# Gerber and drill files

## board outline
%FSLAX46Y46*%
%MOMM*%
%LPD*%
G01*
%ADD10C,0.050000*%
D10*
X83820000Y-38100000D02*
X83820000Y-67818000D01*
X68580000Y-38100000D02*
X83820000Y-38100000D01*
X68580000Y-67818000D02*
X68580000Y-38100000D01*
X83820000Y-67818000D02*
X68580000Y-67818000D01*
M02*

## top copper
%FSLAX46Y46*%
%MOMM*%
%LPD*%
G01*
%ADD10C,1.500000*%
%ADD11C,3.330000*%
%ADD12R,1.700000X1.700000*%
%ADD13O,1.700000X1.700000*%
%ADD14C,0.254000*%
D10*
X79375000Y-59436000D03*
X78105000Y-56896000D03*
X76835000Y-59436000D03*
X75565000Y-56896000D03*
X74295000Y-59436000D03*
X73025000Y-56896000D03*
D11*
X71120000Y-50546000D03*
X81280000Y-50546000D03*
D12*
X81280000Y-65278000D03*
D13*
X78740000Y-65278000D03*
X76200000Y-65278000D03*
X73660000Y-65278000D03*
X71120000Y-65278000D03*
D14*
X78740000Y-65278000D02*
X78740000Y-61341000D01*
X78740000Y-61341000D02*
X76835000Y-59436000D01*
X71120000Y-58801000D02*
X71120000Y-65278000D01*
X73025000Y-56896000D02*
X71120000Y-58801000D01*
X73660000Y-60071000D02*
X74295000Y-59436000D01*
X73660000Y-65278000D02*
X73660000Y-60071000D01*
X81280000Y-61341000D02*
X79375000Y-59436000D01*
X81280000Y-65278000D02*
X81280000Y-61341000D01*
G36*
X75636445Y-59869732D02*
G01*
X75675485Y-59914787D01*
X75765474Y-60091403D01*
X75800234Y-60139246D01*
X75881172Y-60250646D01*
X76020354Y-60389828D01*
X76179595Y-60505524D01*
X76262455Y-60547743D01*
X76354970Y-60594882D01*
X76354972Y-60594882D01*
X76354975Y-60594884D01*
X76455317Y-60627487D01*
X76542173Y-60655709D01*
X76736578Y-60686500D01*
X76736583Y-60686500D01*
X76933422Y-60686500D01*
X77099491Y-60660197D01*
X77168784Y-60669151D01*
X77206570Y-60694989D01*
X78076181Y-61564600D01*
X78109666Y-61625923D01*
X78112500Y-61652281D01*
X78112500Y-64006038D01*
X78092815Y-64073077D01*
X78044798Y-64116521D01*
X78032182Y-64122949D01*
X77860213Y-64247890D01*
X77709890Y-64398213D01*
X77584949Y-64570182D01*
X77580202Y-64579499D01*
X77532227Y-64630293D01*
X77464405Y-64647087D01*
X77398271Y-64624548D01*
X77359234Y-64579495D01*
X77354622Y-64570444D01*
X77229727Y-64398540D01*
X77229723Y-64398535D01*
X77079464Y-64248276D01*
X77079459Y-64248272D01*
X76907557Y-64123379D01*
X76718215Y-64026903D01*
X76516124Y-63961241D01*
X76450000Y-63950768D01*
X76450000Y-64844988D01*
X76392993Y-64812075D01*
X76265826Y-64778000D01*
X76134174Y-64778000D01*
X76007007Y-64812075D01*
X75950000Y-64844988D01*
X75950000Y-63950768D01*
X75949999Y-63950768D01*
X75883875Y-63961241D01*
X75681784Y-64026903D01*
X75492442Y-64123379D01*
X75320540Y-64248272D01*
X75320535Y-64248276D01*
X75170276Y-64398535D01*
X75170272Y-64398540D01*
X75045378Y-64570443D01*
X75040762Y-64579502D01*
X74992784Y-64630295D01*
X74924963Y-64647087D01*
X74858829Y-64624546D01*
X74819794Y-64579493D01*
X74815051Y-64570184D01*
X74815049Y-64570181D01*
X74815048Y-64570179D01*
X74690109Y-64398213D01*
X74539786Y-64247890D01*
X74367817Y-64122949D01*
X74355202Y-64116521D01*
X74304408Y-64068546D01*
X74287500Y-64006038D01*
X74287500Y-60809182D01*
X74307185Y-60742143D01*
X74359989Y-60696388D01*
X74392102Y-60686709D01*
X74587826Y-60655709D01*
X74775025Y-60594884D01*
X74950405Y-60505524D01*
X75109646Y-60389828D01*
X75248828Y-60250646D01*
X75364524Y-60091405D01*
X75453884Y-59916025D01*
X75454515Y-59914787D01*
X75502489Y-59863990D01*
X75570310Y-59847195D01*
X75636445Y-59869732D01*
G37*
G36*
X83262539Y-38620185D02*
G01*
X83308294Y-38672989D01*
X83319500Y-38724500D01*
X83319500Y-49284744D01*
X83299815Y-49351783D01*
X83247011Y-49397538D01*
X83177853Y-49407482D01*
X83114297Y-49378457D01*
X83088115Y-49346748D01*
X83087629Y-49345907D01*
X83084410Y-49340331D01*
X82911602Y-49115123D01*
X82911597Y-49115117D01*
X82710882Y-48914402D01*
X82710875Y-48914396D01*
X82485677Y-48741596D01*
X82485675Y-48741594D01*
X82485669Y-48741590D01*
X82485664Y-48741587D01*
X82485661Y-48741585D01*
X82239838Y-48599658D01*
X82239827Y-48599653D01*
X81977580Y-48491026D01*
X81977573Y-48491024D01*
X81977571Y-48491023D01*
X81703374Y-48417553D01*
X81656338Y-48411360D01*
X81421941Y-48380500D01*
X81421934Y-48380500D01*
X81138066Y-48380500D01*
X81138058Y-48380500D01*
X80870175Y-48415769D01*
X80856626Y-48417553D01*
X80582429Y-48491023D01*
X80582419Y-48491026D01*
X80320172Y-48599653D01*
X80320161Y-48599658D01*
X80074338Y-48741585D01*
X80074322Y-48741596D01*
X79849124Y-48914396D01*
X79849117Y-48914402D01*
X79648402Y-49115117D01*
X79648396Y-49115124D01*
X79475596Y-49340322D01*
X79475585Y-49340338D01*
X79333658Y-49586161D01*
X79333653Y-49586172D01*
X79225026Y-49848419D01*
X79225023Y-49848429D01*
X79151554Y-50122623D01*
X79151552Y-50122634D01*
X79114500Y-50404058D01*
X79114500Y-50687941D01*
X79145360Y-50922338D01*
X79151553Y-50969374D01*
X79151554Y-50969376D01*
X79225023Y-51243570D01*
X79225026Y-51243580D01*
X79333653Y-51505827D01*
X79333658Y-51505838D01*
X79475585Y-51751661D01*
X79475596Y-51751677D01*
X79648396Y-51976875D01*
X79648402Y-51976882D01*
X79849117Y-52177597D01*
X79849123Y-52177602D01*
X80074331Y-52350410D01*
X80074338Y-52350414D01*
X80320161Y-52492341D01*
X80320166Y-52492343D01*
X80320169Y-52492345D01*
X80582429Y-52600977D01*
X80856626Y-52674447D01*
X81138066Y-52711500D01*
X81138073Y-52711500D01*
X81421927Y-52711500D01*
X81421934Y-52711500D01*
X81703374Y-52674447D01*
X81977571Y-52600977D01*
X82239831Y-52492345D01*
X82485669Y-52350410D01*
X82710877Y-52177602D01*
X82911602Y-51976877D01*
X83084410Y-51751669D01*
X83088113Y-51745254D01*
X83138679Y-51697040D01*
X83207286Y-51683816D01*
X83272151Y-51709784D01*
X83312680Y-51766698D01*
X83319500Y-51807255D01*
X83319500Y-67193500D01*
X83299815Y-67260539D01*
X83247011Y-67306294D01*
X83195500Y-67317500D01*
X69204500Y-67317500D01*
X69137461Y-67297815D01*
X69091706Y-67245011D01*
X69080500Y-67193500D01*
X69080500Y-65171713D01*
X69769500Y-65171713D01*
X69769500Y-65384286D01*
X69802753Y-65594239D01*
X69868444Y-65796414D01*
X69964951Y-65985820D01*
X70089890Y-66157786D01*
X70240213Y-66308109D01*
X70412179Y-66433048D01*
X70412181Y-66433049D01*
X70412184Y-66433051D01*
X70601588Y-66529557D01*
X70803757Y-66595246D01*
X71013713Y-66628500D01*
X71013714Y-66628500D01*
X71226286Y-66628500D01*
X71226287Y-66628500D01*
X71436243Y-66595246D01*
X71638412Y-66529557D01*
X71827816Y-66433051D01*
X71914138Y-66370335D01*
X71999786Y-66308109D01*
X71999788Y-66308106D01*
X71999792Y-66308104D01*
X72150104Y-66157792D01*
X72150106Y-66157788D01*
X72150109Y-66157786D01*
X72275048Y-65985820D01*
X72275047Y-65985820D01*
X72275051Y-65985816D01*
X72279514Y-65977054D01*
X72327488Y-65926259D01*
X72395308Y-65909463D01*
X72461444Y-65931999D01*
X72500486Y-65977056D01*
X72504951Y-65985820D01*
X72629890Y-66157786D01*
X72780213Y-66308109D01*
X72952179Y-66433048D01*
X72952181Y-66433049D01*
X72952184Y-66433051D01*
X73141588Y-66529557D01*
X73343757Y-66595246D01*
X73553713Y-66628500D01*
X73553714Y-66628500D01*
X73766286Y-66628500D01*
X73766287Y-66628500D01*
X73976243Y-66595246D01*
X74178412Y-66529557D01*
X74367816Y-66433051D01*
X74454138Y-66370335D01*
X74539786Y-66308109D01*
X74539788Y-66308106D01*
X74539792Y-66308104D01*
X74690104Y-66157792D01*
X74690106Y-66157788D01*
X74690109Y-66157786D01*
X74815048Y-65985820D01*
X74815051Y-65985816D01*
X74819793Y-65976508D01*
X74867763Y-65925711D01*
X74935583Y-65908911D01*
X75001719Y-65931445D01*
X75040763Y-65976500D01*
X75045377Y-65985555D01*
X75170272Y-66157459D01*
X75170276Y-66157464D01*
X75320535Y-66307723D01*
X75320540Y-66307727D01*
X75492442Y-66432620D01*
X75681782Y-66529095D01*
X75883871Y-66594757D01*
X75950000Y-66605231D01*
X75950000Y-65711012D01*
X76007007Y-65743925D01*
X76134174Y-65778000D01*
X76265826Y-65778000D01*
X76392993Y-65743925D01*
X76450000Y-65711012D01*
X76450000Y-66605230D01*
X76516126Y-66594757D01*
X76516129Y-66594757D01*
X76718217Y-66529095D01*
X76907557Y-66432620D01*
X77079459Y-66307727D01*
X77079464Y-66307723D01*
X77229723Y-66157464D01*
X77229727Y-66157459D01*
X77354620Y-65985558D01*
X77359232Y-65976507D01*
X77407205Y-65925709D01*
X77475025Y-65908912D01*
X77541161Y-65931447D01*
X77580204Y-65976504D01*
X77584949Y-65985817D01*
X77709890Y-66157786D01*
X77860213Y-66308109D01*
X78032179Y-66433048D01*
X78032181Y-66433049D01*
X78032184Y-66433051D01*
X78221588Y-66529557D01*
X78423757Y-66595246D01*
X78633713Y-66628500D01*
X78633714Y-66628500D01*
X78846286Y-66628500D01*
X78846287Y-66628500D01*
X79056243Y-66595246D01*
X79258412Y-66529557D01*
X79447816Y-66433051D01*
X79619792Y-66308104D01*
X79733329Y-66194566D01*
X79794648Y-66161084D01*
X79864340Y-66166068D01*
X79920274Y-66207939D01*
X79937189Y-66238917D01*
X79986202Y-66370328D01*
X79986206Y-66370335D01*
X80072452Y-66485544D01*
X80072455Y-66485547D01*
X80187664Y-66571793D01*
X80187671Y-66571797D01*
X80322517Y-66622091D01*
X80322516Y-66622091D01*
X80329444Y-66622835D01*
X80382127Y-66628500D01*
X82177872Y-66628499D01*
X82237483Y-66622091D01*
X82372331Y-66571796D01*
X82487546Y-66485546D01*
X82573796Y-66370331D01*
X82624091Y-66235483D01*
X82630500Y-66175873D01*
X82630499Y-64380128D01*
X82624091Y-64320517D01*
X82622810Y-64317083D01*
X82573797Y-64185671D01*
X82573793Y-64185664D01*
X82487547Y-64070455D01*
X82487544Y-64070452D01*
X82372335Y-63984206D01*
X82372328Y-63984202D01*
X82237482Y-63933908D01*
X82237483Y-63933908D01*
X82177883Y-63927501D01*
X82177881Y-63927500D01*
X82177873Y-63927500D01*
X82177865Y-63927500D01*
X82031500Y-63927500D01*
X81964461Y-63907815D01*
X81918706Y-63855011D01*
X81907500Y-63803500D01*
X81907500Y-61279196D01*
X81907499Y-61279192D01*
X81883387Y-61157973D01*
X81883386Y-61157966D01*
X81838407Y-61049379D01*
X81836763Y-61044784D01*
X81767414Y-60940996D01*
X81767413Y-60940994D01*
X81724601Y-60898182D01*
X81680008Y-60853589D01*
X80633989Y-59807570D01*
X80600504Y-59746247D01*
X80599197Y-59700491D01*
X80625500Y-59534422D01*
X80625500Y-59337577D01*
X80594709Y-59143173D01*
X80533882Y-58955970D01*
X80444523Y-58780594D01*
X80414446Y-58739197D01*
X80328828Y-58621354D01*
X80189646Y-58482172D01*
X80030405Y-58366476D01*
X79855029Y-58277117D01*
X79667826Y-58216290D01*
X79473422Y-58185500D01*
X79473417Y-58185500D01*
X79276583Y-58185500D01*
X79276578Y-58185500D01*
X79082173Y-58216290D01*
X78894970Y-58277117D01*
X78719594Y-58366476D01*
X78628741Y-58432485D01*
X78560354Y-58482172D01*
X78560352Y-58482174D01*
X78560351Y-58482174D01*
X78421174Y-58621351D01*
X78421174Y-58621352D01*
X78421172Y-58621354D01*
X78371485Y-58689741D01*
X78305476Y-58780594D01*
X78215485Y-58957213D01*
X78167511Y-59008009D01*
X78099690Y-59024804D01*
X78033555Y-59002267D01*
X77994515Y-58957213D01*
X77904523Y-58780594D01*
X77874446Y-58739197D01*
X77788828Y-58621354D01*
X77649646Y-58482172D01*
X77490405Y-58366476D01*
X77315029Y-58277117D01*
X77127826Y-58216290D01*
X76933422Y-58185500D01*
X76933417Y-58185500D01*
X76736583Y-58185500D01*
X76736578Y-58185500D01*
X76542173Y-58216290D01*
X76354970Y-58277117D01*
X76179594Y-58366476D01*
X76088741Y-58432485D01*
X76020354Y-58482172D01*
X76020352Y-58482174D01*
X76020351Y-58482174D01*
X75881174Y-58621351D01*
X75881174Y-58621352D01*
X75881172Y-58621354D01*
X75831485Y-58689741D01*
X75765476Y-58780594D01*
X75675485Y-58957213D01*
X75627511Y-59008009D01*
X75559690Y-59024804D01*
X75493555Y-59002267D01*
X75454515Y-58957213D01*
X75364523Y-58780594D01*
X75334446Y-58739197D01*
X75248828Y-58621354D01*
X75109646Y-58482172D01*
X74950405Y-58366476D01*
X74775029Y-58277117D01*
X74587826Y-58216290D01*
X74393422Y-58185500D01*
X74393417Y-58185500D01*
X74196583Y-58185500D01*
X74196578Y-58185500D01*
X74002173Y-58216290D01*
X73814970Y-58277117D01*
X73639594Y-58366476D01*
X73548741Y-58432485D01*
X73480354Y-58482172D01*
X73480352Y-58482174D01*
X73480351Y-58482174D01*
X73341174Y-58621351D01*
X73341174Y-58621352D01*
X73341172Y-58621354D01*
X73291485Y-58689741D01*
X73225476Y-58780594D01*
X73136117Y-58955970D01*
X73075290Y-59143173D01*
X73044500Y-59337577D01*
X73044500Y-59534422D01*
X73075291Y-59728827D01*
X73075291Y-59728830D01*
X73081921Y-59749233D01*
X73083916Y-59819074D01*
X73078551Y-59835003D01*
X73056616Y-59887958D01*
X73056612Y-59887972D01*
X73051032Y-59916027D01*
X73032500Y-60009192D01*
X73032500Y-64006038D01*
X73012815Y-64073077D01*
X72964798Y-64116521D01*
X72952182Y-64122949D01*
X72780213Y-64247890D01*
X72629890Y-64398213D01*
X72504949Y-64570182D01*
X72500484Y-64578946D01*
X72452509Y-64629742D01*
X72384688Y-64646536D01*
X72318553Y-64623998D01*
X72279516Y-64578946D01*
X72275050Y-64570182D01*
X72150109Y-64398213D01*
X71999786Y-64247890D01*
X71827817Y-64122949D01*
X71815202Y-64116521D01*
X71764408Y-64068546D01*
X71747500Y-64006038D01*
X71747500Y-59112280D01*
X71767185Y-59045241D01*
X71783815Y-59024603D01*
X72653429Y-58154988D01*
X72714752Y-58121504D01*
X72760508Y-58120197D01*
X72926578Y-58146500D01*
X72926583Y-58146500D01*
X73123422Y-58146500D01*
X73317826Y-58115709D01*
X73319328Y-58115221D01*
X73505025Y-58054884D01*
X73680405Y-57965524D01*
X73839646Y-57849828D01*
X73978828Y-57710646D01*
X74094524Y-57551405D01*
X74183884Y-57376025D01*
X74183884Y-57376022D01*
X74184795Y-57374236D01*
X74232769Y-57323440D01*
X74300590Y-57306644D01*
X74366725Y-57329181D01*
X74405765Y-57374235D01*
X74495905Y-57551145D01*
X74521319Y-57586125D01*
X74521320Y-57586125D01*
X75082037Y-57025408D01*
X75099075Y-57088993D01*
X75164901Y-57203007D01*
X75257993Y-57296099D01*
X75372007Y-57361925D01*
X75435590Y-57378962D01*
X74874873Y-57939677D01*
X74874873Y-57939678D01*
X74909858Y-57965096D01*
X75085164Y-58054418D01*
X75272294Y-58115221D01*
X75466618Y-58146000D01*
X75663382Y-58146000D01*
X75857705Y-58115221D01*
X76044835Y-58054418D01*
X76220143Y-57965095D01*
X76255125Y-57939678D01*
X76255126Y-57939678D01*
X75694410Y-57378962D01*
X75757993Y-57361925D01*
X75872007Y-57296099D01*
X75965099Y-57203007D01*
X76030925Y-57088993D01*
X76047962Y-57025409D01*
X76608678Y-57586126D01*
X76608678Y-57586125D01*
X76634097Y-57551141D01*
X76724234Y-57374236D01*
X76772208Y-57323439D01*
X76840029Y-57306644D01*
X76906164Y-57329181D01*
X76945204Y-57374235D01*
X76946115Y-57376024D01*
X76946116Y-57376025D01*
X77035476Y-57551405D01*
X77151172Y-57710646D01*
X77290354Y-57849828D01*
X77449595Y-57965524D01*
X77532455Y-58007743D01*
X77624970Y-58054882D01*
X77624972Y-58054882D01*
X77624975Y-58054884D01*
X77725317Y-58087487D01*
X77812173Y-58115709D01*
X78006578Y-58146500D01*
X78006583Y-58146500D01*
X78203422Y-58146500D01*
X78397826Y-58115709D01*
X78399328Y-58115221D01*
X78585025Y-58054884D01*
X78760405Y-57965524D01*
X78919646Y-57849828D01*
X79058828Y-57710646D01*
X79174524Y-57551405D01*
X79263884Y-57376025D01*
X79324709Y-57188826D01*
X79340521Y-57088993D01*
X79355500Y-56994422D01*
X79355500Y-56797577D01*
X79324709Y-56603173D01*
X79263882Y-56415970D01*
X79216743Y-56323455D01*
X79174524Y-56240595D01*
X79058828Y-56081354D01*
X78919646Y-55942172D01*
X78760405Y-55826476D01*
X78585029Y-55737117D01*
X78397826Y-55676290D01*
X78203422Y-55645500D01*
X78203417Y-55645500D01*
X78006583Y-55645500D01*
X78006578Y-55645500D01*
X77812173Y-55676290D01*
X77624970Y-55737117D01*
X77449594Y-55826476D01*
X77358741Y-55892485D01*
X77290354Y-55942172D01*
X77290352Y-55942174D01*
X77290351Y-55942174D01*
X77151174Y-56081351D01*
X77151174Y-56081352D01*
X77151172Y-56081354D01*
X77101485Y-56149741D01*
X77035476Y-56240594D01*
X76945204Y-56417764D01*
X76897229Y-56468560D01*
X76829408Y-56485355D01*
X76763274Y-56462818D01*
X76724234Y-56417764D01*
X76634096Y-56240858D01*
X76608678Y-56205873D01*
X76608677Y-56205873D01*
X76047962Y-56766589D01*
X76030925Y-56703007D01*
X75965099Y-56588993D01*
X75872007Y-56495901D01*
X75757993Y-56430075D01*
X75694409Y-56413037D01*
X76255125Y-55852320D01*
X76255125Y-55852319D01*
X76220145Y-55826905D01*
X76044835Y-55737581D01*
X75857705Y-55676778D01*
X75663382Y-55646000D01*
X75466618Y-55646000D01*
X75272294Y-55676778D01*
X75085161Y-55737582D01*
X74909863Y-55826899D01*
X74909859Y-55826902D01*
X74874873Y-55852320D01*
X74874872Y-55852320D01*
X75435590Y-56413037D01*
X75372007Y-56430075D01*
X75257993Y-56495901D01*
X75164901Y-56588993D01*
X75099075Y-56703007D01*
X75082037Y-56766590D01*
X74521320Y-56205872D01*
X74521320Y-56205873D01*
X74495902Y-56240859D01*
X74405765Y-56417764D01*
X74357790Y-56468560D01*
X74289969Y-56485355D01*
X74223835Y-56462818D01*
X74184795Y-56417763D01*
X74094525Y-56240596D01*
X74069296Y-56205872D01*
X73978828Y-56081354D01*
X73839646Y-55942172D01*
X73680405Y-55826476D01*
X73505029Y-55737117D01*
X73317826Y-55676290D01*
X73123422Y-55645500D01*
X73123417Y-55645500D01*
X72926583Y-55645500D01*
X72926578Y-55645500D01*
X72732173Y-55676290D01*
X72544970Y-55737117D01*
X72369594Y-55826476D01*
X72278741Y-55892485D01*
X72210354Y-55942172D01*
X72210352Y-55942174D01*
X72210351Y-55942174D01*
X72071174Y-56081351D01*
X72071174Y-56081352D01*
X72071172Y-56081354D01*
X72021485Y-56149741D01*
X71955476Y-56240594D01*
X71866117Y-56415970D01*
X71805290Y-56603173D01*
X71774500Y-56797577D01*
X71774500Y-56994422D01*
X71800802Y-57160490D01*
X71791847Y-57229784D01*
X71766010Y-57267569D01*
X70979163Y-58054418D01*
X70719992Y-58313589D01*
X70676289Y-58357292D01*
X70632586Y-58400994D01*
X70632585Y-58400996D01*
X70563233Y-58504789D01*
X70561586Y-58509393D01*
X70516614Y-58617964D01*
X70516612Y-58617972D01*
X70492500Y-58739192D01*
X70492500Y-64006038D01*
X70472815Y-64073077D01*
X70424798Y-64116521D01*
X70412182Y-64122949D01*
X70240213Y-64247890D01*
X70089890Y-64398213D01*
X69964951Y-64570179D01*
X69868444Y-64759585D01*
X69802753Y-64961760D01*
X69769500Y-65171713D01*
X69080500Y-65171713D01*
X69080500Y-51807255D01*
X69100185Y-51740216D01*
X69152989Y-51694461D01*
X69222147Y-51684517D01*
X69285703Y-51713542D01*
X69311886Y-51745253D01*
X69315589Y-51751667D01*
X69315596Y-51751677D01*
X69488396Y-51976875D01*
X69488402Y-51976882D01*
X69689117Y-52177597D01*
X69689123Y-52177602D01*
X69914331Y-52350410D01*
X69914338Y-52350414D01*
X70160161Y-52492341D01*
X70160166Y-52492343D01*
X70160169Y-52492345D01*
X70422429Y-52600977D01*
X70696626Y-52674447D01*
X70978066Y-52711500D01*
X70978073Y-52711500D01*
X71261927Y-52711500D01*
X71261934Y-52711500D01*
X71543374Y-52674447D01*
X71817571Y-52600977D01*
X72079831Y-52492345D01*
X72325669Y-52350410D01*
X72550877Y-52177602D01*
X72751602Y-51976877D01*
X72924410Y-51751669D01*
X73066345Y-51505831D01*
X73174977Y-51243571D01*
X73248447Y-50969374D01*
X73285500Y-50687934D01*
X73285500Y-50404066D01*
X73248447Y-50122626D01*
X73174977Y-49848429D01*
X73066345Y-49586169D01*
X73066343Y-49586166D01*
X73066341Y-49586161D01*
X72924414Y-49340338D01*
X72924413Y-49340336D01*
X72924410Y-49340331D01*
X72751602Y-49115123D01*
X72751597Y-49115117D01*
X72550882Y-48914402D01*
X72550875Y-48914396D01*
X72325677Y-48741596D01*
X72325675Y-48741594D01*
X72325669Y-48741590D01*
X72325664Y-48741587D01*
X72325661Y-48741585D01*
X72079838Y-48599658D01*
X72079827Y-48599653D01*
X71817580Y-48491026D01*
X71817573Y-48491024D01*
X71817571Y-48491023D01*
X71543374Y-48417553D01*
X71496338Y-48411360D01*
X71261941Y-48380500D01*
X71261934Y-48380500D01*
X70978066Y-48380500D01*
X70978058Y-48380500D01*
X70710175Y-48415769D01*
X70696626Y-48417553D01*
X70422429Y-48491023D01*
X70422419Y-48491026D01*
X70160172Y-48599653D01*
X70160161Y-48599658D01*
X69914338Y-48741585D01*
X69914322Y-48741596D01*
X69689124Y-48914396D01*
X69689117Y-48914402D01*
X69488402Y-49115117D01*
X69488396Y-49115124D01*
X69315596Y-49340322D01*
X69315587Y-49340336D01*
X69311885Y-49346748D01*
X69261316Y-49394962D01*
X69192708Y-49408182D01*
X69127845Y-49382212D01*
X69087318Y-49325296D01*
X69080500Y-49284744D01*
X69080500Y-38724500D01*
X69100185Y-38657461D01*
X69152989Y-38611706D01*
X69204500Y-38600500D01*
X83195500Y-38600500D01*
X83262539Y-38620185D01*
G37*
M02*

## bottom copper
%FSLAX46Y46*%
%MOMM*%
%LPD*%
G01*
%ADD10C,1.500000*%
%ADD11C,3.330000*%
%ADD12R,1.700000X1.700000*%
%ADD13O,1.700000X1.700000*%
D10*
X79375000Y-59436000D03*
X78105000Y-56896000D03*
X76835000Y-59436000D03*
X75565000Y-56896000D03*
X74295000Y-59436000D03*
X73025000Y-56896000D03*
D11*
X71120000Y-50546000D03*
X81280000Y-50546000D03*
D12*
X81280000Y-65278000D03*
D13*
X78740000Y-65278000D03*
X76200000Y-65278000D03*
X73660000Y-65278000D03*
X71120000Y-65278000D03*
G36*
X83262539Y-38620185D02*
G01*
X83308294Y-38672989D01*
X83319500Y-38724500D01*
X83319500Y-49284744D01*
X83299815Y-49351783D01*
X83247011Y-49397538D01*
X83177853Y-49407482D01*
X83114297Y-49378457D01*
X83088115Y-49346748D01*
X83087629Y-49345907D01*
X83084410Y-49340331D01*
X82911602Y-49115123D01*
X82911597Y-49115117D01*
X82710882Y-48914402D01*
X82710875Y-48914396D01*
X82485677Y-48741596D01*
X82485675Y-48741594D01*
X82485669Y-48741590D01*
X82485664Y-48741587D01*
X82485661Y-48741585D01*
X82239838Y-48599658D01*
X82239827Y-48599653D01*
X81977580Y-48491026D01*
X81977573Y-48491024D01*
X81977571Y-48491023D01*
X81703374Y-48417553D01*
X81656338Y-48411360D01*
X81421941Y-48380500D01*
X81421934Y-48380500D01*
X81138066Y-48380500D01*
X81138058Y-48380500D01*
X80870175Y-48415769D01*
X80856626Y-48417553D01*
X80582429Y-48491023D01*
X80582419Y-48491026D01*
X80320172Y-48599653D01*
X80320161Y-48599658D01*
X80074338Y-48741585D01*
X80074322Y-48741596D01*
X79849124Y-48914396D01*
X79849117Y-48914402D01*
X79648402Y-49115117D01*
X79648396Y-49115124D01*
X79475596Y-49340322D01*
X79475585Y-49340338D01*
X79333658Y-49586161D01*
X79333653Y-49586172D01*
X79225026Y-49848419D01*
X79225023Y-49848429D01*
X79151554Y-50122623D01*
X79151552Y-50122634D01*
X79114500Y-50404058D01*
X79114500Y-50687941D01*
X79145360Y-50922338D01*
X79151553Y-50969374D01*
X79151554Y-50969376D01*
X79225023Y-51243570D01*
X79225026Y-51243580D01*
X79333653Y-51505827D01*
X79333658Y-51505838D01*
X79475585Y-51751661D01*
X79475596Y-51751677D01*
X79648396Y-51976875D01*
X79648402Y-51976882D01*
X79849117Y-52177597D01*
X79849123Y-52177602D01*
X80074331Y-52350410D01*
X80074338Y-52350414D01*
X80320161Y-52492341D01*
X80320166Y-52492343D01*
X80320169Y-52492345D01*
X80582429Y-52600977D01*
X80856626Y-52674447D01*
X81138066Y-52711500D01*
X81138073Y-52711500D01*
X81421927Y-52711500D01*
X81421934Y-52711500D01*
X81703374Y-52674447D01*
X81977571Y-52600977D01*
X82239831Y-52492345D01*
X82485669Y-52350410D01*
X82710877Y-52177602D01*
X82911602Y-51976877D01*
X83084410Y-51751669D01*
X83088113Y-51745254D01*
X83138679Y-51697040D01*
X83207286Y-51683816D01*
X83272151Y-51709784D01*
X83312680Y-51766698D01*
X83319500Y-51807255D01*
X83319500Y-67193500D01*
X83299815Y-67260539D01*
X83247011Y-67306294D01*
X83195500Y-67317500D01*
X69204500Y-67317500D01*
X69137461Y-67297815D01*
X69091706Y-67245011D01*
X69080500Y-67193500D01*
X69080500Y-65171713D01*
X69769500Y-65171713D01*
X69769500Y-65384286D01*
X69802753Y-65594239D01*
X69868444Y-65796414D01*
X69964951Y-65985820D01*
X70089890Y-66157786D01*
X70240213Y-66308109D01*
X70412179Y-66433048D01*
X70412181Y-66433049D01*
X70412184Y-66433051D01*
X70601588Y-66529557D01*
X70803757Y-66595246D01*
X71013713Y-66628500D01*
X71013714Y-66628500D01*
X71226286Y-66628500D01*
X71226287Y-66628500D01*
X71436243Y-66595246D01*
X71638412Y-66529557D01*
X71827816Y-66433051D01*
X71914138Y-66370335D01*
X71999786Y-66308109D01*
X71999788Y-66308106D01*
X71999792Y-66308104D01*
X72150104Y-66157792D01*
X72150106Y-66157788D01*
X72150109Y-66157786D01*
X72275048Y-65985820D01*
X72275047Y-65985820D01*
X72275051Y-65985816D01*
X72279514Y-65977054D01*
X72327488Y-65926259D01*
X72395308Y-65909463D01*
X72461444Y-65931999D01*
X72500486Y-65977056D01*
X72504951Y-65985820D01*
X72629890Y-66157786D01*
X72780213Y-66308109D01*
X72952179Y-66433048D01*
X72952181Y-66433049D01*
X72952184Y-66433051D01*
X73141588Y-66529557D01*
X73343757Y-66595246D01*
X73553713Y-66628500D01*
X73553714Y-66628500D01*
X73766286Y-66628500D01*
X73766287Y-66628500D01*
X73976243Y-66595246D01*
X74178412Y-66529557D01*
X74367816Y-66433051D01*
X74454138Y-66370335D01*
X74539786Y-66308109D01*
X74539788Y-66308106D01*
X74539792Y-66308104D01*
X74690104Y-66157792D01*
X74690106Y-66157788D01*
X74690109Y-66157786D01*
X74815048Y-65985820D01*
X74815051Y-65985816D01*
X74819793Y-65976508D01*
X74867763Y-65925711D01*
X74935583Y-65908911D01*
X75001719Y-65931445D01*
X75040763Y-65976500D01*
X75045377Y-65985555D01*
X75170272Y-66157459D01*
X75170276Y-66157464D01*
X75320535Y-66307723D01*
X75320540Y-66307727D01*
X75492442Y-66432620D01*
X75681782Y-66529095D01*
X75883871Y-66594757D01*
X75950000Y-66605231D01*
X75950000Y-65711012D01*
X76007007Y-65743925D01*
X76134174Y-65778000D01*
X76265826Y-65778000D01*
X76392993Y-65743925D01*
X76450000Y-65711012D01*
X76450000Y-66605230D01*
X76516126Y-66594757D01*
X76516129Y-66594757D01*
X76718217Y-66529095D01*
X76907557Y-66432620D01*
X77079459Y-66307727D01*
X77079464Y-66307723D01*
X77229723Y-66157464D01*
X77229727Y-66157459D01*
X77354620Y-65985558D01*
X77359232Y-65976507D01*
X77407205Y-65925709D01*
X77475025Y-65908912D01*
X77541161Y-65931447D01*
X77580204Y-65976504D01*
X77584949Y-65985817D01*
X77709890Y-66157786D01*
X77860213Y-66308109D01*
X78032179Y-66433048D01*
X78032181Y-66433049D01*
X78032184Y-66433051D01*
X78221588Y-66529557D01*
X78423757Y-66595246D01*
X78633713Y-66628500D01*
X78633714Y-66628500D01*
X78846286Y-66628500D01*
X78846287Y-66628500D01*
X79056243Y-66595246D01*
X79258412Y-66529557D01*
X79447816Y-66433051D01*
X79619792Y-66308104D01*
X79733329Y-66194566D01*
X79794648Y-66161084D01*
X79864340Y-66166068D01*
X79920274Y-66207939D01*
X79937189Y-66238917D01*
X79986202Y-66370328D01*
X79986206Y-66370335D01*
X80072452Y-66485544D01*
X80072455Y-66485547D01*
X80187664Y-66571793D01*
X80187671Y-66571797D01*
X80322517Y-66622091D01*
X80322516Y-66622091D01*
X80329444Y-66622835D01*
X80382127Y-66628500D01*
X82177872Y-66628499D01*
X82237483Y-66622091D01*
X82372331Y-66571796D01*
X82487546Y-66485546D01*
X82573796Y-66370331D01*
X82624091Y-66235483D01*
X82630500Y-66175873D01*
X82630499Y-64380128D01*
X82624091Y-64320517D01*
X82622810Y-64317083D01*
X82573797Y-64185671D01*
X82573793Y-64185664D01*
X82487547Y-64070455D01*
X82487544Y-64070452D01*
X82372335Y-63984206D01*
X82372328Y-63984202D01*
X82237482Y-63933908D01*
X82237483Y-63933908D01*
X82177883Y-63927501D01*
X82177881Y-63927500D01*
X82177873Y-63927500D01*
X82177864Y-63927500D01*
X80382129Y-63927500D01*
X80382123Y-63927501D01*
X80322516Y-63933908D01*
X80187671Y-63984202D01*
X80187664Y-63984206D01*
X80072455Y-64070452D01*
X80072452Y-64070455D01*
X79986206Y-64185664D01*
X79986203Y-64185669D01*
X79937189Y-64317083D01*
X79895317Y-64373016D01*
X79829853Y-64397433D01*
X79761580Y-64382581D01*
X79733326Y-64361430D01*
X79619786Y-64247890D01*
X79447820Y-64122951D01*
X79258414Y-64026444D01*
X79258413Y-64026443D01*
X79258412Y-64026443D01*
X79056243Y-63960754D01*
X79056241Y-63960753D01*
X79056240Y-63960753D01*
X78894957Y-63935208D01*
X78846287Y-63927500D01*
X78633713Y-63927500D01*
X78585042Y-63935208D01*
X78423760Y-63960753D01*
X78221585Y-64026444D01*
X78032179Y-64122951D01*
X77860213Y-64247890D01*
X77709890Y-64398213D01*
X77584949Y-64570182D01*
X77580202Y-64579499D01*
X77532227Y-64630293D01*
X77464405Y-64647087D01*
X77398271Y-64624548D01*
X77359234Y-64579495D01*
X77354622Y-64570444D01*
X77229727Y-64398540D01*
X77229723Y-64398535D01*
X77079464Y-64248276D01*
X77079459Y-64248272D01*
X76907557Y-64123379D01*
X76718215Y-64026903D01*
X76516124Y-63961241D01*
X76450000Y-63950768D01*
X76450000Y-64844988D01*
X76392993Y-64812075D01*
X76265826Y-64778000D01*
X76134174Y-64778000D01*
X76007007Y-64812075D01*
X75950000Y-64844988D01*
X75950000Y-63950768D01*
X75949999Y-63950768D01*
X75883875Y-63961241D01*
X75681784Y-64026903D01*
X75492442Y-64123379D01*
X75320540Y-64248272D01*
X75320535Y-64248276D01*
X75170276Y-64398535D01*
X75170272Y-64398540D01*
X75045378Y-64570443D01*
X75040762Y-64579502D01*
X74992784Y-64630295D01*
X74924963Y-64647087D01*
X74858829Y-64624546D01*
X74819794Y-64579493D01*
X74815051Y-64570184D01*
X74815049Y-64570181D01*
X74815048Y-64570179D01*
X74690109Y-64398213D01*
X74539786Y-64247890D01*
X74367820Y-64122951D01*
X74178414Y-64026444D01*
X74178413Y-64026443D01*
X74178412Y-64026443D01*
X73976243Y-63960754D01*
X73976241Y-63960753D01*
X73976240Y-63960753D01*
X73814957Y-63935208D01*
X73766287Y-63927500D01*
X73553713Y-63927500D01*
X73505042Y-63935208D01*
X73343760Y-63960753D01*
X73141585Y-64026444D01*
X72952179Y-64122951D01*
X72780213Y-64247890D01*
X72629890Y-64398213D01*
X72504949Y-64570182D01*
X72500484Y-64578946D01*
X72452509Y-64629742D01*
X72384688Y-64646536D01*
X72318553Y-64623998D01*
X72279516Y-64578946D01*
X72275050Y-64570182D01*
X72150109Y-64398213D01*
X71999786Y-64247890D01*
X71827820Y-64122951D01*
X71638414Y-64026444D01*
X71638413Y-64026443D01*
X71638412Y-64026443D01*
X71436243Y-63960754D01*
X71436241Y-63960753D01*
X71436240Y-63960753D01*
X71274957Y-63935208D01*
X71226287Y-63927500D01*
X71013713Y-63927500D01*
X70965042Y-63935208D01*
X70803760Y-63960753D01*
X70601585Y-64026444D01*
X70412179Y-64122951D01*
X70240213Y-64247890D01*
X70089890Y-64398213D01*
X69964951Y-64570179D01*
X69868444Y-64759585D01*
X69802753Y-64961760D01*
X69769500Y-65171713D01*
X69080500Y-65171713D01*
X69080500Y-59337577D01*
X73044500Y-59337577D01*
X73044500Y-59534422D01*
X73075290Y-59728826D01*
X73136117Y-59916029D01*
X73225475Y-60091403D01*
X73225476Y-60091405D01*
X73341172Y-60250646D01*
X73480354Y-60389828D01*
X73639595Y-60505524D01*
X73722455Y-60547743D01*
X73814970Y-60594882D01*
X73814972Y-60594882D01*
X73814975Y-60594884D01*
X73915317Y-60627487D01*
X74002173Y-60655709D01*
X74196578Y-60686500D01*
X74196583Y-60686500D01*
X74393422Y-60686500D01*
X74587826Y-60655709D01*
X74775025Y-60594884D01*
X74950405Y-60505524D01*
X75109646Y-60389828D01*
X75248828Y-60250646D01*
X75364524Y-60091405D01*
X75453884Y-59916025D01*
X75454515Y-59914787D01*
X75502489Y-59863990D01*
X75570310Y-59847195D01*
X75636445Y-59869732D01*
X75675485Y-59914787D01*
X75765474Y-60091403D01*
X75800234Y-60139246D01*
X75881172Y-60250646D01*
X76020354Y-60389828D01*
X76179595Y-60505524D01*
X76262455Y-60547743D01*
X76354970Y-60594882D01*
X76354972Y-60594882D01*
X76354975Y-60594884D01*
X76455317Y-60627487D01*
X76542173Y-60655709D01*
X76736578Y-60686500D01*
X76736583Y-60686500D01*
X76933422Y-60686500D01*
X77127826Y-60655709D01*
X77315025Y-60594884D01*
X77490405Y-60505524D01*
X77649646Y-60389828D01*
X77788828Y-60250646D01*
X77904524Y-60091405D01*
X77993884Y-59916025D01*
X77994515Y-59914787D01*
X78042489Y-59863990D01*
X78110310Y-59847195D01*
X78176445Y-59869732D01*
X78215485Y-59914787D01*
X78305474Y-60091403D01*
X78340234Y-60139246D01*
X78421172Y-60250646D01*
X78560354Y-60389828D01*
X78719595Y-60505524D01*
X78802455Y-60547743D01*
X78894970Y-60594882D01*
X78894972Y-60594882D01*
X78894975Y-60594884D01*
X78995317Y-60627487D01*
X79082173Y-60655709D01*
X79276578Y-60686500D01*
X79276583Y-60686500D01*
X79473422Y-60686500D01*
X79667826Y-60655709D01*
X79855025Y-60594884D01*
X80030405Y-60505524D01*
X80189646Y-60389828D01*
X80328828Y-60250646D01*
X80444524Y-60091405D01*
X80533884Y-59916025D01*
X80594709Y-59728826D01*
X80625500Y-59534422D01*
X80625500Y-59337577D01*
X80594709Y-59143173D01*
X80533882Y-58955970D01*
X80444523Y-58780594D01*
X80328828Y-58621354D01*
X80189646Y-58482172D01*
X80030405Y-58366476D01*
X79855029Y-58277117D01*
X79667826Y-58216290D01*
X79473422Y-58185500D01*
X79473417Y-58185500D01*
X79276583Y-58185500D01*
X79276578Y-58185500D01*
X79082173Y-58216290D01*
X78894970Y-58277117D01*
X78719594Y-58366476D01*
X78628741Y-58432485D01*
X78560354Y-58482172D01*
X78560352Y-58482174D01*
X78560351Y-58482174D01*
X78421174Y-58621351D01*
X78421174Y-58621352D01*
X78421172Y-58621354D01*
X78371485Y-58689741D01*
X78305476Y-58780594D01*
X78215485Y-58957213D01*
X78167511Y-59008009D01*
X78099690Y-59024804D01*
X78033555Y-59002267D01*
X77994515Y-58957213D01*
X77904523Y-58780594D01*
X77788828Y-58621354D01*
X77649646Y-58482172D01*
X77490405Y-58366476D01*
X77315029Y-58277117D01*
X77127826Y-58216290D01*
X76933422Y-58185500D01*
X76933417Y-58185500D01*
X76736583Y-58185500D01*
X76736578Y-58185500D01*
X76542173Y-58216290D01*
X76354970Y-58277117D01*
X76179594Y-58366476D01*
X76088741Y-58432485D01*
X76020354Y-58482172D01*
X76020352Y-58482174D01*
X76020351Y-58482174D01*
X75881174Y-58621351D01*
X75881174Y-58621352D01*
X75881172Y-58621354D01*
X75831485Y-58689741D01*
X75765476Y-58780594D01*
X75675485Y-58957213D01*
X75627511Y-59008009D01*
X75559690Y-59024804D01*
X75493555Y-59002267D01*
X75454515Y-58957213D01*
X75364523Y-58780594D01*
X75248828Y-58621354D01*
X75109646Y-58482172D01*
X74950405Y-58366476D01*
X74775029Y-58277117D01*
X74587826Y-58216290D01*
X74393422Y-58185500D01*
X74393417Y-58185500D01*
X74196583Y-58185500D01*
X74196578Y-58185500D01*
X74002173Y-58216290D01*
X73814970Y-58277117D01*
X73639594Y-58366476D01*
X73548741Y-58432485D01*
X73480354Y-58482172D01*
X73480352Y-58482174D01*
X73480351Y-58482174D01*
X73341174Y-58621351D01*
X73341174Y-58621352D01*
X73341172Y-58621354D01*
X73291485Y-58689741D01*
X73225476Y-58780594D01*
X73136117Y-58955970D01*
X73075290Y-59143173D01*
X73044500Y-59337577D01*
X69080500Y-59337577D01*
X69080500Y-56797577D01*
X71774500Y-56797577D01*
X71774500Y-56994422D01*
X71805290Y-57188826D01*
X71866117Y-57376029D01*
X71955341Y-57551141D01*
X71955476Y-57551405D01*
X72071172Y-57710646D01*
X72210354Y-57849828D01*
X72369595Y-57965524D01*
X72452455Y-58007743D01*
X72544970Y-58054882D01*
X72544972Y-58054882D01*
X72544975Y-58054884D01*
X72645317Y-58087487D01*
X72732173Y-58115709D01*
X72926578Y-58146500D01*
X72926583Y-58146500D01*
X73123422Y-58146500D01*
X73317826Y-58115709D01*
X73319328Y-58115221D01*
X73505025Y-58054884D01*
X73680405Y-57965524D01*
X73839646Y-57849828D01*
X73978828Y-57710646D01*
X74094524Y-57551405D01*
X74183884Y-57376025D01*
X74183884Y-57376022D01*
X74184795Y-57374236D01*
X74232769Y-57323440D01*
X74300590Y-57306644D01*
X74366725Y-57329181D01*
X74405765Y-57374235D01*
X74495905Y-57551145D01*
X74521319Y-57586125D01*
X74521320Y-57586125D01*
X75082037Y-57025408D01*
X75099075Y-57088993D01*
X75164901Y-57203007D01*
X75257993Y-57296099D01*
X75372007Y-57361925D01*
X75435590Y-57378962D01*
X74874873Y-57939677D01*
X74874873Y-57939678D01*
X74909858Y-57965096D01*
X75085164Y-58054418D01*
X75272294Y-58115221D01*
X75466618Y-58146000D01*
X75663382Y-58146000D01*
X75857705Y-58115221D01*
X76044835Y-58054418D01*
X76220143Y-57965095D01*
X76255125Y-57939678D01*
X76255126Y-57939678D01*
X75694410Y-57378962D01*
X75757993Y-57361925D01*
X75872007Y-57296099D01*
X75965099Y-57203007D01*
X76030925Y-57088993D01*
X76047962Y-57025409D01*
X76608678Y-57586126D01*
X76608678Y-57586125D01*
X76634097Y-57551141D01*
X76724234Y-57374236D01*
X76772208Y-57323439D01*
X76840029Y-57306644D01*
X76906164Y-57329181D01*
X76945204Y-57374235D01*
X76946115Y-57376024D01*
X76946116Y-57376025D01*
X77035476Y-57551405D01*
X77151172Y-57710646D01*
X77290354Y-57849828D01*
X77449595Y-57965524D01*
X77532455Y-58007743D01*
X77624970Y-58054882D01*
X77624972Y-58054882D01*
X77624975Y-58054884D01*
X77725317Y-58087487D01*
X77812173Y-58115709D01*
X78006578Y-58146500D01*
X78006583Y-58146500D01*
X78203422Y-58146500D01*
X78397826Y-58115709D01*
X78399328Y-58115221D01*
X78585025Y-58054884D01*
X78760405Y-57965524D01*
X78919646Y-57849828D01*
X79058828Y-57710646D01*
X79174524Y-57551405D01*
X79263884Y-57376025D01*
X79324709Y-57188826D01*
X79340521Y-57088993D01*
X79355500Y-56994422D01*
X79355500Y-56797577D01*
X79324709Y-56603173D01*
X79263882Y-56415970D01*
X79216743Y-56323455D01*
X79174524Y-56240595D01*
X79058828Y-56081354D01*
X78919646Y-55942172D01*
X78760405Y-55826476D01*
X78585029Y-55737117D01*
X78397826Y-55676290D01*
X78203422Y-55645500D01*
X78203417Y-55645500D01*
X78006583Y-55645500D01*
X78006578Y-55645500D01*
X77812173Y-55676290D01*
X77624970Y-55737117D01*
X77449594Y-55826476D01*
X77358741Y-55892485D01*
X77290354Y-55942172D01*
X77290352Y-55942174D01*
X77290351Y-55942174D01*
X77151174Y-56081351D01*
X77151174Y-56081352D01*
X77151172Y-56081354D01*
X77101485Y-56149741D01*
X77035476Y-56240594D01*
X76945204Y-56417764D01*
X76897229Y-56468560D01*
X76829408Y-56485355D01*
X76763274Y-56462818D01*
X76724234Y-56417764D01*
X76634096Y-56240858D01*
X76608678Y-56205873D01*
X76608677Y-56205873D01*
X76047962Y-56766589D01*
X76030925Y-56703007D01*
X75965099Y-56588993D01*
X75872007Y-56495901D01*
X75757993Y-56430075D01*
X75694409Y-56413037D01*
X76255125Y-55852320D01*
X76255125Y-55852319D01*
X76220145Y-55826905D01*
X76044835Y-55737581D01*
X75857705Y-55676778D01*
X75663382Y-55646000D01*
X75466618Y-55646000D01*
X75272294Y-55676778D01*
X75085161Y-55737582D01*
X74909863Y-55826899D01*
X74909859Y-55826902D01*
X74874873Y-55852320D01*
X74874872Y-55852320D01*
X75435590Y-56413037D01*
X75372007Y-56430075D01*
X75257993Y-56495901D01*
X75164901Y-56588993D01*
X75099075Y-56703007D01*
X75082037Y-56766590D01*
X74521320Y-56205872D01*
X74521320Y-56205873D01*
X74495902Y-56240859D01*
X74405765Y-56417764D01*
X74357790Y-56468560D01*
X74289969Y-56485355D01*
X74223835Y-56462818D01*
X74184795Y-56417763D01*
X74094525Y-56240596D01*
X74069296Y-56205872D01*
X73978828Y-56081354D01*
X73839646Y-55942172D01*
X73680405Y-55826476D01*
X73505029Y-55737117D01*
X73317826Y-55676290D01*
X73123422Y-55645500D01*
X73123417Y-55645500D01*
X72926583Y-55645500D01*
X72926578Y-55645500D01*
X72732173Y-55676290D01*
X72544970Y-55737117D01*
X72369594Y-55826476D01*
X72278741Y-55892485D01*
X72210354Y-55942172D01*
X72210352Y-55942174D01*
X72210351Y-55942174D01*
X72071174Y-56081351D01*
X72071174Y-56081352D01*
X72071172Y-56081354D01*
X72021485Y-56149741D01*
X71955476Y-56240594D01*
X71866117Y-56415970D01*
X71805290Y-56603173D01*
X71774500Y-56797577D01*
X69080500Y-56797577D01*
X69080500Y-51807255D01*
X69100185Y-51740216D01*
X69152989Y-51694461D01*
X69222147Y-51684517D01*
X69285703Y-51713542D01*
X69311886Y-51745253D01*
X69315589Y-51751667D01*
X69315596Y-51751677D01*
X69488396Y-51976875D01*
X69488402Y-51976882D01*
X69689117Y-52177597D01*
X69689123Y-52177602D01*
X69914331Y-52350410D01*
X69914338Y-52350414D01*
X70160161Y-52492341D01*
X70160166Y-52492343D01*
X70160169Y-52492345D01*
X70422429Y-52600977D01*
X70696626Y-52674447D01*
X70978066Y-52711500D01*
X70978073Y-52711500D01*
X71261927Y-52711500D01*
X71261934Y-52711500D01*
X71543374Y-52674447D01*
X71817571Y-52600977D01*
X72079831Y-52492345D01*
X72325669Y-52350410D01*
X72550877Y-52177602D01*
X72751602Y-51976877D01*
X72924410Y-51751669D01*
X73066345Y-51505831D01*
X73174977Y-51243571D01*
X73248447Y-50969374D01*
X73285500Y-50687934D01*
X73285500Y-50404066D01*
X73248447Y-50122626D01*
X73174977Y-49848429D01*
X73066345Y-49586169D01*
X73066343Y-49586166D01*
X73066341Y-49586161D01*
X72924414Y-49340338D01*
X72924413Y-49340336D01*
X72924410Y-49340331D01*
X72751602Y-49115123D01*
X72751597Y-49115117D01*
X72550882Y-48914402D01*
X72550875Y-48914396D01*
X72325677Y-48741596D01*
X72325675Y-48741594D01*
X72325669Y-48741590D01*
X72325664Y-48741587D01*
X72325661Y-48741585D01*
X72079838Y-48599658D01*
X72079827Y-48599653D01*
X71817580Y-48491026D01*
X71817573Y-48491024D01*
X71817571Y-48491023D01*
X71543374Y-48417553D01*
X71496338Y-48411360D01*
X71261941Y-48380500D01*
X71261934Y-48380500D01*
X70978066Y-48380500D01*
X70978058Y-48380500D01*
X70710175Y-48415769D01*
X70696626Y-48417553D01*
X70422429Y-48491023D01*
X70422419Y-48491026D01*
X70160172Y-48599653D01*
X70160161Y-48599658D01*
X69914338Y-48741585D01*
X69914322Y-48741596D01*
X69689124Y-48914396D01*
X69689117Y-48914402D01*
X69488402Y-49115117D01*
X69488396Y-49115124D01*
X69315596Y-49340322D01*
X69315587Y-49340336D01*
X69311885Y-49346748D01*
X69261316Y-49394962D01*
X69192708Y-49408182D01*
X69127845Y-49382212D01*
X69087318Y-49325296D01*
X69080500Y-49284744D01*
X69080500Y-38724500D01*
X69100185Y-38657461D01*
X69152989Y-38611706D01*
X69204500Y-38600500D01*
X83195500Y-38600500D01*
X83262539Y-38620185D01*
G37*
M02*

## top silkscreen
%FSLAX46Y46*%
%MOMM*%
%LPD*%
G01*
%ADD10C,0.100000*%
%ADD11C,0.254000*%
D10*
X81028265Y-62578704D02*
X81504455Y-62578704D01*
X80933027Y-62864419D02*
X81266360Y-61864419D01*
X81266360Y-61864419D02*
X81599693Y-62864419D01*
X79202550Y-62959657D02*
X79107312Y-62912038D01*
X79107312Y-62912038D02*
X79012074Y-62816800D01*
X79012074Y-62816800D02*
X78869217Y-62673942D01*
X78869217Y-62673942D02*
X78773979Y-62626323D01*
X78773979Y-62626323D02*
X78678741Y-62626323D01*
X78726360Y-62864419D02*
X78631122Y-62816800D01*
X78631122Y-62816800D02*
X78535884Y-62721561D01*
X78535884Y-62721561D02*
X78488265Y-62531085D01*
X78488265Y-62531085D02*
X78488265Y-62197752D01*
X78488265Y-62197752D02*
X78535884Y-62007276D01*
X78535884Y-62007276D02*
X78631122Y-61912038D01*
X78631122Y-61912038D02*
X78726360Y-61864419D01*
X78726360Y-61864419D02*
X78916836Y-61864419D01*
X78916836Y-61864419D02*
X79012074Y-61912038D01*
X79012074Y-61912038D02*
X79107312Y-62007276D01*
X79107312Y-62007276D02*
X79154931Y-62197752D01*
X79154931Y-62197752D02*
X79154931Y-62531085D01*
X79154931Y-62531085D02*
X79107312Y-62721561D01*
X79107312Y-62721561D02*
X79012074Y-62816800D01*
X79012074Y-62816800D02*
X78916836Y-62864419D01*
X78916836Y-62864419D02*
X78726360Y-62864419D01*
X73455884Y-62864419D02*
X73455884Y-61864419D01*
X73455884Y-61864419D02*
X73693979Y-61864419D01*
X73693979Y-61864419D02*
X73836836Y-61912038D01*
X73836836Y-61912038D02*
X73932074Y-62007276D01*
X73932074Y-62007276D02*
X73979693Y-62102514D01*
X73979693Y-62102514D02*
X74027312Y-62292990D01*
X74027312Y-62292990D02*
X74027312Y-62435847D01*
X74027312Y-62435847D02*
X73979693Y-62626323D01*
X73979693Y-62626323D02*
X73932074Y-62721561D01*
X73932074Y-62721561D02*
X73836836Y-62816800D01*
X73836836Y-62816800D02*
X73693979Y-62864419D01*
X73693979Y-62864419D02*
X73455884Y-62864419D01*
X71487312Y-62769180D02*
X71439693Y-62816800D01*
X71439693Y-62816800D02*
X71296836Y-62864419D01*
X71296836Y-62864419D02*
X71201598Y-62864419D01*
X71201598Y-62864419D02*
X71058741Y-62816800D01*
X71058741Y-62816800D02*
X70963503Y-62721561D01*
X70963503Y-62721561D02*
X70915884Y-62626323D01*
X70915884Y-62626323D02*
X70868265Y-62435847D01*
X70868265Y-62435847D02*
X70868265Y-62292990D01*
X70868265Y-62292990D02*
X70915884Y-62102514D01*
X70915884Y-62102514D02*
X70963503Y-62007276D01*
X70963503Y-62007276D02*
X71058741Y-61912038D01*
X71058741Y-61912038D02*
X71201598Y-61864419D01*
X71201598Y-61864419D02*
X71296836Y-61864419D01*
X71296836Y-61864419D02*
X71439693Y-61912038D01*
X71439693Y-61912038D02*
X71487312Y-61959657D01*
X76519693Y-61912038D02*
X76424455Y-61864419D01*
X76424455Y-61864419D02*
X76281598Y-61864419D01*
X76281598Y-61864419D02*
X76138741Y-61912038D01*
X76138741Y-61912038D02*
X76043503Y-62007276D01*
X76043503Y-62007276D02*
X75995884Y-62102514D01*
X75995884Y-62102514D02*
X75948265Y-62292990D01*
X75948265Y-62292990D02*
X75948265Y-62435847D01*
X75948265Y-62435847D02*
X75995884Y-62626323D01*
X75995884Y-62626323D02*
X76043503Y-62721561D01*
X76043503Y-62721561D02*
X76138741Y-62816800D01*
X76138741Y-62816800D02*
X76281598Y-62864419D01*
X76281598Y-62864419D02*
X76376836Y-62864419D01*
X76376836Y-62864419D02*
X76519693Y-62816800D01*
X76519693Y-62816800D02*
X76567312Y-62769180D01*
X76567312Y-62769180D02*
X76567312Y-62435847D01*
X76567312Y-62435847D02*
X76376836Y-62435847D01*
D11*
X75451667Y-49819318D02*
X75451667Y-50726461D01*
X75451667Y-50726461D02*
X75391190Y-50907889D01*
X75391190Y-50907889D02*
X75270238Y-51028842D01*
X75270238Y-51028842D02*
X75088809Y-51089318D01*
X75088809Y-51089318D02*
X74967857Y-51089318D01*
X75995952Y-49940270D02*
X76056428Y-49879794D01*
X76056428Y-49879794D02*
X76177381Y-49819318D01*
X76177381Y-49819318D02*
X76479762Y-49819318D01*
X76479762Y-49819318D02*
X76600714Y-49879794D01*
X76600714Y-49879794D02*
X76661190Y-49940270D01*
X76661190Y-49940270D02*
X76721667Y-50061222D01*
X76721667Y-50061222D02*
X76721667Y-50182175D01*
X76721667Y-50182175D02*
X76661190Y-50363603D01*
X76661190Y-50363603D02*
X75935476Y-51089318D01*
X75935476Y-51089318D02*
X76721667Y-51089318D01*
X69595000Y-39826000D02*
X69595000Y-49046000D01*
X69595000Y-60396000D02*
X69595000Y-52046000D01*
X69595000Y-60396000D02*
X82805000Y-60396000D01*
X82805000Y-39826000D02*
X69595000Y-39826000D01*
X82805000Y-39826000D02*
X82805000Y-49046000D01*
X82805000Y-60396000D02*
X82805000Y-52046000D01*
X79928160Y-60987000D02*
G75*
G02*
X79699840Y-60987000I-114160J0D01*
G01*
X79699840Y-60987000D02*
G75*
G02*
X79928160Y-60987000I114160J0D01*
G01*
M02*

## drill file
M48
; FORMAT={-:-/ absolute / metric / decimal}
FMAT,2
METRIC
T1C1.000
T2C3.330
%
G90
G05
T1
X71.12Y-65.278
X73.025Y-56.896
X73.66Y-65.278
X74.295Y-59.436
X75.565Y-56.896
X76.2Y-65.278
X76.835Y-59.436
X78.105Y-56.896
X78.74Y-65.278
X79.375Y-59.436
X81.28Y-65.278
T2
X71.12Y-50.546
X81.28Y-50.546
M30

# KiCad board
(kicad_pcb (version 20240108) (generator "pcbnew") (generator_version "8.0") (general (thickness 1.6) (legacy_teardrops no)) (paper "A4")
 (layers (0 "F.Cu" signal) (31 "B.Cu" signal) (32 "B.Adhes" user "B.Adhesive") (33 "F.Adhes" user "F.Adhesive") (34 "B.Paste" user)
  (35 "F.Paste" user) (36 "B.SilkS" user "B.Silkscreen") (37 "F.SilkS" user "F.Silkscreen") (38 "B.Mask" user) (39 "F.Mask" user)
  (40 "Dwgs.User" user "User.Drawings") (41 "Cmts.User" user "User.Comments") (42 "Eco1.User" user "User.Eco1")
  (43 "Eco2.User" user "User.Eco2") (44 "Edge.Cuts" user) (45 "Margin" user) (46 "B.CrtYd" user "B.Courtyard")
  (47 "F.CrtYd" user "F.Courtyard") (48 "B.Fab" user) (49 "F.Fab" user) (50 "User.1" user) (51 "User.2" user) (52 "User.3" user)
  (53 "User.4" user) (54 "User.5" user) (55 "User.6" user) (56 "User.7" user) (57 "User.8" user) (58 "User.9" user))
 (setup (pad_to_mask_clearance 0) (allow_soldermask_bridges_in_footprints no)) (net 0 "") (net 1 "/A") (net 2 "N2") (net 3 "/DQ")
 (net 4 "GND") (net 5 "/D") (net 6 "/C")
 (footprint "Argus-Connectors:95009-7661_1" (layer "F.Cu") (at 76.2 50.546)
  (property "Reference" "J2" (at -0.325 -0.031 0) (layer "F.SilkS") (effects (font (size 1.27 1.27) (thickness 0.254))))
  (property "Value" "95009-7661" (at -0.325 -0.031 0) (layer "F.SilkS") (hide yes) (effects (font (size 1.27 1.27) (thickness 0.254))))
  (fp_line (start -6.605 -10.72) (end -6.605 -1.5) (stroke (width 0.254) (type solid)) (layer "F.SilkS"))
  (fp_line (start -6.605 9.85) (end -6.605 1.5) (stroke (width 0.254) (type solid)) (layer "F.SilkS"))
  (fp_line (start -6.605 9.85) (end 6.605 9.85) (stroke (width 0.254) (type solid)) (layer "F.SilkS"))
  (fp_line (start 6.605 -10.72) (end -6.605 -10.72) (stroke (width 0.254) (type solid)) (layer "F.SilkS"))
  (fp_line (start 6.605 -10.72) (end 6.605 -1.5) (stroke (width 0.254) (type solid)) (layer "F.SilkS"))
  (fp_line (start 6.605 9.85) (end 6.605 1.5) (stroke (width 0.254) (type solid)) (layer "F.SilkS"))
  (fp_circle (center 3.614 10.441) (end 3.614 10.55516) (stroke (width 0.254) (type solid)) (fill none) (layer "F.SilkS"))
  (pad "1" thru_hole circle (at 3.175 8.89) (size 1.5 1.5) (drill 1) (layers "*.Cu" "*.Mask") (remove_unused_layers no) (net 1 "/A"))
  (pad "2" thru_hole circle (at 1.905 6.35) (size 1.5 1.5) (drill 1) (layers "*.Cu" "*.Mask") (remove_unused_layers no) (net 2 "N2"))
  (pad "3" thru_hole circle (at 0.635 8.89) (size 1.5 1.5) (drill 1) (layers "*.Cu" "*.Mask") (remove_unused_layers no) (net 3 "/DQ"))
  (pad "4" thru_hole circle (at -0.635 6.35) (size 1.5 1.5) (drill 1) (layers "*.Cu" "*.Mask") (remove_unused_layers no) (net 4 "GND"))
  (pad "5" thru_hole circle (at -1.905 8.89) (size 1.5 1.5) (drill 1) (layers "*.Cu" "*.Mask") (remove_unused_layers no) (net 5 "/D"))
  (pad "6" thru_hole circle (at -3.175 6.35) (size 1.5 1.5) (drill 1) (layers "*.Cu" "*.Mask") (remove_unused_layers no) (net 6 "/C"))
  (pad "7" thru_hole circle (at -5.08 0) (size 3.33 3.33) (drill 3.33) (layers "*.Cu" "*.Mask") (remove_unused_layers no))
  (pad "8" thru_hole circle (at 5.08 0) (size 3.33 3.33) (drill 3.33) (layers "*.Cu" "*.Mask") (remove_unused_layers no)))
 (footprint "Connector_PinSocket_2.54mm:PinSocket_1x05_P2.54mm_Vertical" (layer "B.Cu") (at 81.28 65.278 90)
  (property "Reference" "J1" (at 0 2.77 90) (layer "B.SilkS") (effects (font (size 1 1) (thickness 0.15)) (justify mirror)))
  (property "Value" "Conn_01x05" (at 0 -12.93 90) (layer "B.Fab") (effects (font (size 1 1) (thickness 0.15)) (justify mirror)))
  (pad "1" thru_hole rect (at 0 0 90) (size 1.7 1.7) (drill 1) (layers "*.Cu" "*.Mask") (remove_unused_layers no) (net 1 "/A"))
  (pad "2" thru_hole oval (at 0 -2.54 90) (size 1.7 1.7) (drill 1) (layers "*.Cu" "*.Mask") (remove_unused_layers no) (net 3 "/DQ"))
  (pad "3" thru_hole oval (at 0 -5.08 90) (size 1.7 1.7) (drill 1) (layers "*.Cu" "*.Mask") (remove_unused_layers no) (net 4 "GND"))
  (pad "4" thru_hole oval (at 0 -7.62 90) (size 1.7 1.7) (drill 1) (layers "*.Cu" "*.Mask") (remove_unused_layers no) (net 5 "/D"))
  (pad "5" thru_hole oval (at 0 -10.16 90) (size 1.7 1.7) (drill 1) (layers "*.Cu" "*.Mask") (remove_unused_layers no) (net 6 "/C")))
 (gr_line (start 83.82 38.1) (end 83.82 67.818) (stroke (width 0.05) (type default)) (layer "Edge.Cuts"))
 (gr_line (start 68.58 38.1) (end 83.82 38.1) (stroke (width 0.05) (type default)) (layer "Edge.Cuts"))
 (gr_line (start 68.58 67.818) (end 68.58 38.1) (stroke (width 0.05) (type default)) (layer "Edge.Cuts"))
 (gr_line (start 83.82 67.818) (end 68.58 67.818) (stroke (width 0.05) (type default)) (layer "Edge.Cuts"))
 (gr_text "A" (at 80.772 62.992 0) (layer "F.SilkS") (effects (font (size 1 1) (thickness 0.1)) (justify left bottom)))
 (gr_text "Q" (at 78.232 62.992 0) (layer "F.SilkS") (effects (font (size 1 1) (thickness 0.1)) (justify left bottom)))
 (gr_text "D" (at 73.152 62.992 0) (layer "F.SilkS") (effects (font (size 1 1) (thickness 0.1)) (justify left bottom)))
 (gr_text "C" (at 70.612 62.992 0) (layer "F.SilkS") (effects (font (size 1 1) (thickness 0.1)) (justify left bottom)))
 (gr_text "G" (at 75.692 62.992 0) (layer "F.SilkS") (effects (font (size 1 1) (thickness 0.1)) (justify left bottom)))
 (segment (start 78.74 65.278) (end 78.74 61.341) (width 0.254) (layer "F.Cu") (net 3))
 (segment (start 78.74 61.341) (end 76.835 59.436) (width 0.254) (layer "F.Cu") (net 3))
 (segment (start 71.12 58.801) (end 71.12 65.278) (width 0.254) (layer "F.Cu") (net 6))
 (segment (start 73.025 56.896) (end 71.12 58.801) (width 0.254) (layer "F.Cu") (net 6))
 (segment (start 73.66 60.071) (end 74.295 59.436) (width 0.254) (layer "F.Cu") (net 5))
 (segment (start 73.66 65.278) (end 73.66 60.071) (width 0.254) (layer "F.Cu") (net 5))
 (segment (start 81.28 61.341) (end 79.375 59.436) (width 0.254) (layer "F.Cu") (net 1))
 (segment (start 81.28 65.278) (end 81.28 61.341) (width 0.254) (layer "F.Cu") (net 1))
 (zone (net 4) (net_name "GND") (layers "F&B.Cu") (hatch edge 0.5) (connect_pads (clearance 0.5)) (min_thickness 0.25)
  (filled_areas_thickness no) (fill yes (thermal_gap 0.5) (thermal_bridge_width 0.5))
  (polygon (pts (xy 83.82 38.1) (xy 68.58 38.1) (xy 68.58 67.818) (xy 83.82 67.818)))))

